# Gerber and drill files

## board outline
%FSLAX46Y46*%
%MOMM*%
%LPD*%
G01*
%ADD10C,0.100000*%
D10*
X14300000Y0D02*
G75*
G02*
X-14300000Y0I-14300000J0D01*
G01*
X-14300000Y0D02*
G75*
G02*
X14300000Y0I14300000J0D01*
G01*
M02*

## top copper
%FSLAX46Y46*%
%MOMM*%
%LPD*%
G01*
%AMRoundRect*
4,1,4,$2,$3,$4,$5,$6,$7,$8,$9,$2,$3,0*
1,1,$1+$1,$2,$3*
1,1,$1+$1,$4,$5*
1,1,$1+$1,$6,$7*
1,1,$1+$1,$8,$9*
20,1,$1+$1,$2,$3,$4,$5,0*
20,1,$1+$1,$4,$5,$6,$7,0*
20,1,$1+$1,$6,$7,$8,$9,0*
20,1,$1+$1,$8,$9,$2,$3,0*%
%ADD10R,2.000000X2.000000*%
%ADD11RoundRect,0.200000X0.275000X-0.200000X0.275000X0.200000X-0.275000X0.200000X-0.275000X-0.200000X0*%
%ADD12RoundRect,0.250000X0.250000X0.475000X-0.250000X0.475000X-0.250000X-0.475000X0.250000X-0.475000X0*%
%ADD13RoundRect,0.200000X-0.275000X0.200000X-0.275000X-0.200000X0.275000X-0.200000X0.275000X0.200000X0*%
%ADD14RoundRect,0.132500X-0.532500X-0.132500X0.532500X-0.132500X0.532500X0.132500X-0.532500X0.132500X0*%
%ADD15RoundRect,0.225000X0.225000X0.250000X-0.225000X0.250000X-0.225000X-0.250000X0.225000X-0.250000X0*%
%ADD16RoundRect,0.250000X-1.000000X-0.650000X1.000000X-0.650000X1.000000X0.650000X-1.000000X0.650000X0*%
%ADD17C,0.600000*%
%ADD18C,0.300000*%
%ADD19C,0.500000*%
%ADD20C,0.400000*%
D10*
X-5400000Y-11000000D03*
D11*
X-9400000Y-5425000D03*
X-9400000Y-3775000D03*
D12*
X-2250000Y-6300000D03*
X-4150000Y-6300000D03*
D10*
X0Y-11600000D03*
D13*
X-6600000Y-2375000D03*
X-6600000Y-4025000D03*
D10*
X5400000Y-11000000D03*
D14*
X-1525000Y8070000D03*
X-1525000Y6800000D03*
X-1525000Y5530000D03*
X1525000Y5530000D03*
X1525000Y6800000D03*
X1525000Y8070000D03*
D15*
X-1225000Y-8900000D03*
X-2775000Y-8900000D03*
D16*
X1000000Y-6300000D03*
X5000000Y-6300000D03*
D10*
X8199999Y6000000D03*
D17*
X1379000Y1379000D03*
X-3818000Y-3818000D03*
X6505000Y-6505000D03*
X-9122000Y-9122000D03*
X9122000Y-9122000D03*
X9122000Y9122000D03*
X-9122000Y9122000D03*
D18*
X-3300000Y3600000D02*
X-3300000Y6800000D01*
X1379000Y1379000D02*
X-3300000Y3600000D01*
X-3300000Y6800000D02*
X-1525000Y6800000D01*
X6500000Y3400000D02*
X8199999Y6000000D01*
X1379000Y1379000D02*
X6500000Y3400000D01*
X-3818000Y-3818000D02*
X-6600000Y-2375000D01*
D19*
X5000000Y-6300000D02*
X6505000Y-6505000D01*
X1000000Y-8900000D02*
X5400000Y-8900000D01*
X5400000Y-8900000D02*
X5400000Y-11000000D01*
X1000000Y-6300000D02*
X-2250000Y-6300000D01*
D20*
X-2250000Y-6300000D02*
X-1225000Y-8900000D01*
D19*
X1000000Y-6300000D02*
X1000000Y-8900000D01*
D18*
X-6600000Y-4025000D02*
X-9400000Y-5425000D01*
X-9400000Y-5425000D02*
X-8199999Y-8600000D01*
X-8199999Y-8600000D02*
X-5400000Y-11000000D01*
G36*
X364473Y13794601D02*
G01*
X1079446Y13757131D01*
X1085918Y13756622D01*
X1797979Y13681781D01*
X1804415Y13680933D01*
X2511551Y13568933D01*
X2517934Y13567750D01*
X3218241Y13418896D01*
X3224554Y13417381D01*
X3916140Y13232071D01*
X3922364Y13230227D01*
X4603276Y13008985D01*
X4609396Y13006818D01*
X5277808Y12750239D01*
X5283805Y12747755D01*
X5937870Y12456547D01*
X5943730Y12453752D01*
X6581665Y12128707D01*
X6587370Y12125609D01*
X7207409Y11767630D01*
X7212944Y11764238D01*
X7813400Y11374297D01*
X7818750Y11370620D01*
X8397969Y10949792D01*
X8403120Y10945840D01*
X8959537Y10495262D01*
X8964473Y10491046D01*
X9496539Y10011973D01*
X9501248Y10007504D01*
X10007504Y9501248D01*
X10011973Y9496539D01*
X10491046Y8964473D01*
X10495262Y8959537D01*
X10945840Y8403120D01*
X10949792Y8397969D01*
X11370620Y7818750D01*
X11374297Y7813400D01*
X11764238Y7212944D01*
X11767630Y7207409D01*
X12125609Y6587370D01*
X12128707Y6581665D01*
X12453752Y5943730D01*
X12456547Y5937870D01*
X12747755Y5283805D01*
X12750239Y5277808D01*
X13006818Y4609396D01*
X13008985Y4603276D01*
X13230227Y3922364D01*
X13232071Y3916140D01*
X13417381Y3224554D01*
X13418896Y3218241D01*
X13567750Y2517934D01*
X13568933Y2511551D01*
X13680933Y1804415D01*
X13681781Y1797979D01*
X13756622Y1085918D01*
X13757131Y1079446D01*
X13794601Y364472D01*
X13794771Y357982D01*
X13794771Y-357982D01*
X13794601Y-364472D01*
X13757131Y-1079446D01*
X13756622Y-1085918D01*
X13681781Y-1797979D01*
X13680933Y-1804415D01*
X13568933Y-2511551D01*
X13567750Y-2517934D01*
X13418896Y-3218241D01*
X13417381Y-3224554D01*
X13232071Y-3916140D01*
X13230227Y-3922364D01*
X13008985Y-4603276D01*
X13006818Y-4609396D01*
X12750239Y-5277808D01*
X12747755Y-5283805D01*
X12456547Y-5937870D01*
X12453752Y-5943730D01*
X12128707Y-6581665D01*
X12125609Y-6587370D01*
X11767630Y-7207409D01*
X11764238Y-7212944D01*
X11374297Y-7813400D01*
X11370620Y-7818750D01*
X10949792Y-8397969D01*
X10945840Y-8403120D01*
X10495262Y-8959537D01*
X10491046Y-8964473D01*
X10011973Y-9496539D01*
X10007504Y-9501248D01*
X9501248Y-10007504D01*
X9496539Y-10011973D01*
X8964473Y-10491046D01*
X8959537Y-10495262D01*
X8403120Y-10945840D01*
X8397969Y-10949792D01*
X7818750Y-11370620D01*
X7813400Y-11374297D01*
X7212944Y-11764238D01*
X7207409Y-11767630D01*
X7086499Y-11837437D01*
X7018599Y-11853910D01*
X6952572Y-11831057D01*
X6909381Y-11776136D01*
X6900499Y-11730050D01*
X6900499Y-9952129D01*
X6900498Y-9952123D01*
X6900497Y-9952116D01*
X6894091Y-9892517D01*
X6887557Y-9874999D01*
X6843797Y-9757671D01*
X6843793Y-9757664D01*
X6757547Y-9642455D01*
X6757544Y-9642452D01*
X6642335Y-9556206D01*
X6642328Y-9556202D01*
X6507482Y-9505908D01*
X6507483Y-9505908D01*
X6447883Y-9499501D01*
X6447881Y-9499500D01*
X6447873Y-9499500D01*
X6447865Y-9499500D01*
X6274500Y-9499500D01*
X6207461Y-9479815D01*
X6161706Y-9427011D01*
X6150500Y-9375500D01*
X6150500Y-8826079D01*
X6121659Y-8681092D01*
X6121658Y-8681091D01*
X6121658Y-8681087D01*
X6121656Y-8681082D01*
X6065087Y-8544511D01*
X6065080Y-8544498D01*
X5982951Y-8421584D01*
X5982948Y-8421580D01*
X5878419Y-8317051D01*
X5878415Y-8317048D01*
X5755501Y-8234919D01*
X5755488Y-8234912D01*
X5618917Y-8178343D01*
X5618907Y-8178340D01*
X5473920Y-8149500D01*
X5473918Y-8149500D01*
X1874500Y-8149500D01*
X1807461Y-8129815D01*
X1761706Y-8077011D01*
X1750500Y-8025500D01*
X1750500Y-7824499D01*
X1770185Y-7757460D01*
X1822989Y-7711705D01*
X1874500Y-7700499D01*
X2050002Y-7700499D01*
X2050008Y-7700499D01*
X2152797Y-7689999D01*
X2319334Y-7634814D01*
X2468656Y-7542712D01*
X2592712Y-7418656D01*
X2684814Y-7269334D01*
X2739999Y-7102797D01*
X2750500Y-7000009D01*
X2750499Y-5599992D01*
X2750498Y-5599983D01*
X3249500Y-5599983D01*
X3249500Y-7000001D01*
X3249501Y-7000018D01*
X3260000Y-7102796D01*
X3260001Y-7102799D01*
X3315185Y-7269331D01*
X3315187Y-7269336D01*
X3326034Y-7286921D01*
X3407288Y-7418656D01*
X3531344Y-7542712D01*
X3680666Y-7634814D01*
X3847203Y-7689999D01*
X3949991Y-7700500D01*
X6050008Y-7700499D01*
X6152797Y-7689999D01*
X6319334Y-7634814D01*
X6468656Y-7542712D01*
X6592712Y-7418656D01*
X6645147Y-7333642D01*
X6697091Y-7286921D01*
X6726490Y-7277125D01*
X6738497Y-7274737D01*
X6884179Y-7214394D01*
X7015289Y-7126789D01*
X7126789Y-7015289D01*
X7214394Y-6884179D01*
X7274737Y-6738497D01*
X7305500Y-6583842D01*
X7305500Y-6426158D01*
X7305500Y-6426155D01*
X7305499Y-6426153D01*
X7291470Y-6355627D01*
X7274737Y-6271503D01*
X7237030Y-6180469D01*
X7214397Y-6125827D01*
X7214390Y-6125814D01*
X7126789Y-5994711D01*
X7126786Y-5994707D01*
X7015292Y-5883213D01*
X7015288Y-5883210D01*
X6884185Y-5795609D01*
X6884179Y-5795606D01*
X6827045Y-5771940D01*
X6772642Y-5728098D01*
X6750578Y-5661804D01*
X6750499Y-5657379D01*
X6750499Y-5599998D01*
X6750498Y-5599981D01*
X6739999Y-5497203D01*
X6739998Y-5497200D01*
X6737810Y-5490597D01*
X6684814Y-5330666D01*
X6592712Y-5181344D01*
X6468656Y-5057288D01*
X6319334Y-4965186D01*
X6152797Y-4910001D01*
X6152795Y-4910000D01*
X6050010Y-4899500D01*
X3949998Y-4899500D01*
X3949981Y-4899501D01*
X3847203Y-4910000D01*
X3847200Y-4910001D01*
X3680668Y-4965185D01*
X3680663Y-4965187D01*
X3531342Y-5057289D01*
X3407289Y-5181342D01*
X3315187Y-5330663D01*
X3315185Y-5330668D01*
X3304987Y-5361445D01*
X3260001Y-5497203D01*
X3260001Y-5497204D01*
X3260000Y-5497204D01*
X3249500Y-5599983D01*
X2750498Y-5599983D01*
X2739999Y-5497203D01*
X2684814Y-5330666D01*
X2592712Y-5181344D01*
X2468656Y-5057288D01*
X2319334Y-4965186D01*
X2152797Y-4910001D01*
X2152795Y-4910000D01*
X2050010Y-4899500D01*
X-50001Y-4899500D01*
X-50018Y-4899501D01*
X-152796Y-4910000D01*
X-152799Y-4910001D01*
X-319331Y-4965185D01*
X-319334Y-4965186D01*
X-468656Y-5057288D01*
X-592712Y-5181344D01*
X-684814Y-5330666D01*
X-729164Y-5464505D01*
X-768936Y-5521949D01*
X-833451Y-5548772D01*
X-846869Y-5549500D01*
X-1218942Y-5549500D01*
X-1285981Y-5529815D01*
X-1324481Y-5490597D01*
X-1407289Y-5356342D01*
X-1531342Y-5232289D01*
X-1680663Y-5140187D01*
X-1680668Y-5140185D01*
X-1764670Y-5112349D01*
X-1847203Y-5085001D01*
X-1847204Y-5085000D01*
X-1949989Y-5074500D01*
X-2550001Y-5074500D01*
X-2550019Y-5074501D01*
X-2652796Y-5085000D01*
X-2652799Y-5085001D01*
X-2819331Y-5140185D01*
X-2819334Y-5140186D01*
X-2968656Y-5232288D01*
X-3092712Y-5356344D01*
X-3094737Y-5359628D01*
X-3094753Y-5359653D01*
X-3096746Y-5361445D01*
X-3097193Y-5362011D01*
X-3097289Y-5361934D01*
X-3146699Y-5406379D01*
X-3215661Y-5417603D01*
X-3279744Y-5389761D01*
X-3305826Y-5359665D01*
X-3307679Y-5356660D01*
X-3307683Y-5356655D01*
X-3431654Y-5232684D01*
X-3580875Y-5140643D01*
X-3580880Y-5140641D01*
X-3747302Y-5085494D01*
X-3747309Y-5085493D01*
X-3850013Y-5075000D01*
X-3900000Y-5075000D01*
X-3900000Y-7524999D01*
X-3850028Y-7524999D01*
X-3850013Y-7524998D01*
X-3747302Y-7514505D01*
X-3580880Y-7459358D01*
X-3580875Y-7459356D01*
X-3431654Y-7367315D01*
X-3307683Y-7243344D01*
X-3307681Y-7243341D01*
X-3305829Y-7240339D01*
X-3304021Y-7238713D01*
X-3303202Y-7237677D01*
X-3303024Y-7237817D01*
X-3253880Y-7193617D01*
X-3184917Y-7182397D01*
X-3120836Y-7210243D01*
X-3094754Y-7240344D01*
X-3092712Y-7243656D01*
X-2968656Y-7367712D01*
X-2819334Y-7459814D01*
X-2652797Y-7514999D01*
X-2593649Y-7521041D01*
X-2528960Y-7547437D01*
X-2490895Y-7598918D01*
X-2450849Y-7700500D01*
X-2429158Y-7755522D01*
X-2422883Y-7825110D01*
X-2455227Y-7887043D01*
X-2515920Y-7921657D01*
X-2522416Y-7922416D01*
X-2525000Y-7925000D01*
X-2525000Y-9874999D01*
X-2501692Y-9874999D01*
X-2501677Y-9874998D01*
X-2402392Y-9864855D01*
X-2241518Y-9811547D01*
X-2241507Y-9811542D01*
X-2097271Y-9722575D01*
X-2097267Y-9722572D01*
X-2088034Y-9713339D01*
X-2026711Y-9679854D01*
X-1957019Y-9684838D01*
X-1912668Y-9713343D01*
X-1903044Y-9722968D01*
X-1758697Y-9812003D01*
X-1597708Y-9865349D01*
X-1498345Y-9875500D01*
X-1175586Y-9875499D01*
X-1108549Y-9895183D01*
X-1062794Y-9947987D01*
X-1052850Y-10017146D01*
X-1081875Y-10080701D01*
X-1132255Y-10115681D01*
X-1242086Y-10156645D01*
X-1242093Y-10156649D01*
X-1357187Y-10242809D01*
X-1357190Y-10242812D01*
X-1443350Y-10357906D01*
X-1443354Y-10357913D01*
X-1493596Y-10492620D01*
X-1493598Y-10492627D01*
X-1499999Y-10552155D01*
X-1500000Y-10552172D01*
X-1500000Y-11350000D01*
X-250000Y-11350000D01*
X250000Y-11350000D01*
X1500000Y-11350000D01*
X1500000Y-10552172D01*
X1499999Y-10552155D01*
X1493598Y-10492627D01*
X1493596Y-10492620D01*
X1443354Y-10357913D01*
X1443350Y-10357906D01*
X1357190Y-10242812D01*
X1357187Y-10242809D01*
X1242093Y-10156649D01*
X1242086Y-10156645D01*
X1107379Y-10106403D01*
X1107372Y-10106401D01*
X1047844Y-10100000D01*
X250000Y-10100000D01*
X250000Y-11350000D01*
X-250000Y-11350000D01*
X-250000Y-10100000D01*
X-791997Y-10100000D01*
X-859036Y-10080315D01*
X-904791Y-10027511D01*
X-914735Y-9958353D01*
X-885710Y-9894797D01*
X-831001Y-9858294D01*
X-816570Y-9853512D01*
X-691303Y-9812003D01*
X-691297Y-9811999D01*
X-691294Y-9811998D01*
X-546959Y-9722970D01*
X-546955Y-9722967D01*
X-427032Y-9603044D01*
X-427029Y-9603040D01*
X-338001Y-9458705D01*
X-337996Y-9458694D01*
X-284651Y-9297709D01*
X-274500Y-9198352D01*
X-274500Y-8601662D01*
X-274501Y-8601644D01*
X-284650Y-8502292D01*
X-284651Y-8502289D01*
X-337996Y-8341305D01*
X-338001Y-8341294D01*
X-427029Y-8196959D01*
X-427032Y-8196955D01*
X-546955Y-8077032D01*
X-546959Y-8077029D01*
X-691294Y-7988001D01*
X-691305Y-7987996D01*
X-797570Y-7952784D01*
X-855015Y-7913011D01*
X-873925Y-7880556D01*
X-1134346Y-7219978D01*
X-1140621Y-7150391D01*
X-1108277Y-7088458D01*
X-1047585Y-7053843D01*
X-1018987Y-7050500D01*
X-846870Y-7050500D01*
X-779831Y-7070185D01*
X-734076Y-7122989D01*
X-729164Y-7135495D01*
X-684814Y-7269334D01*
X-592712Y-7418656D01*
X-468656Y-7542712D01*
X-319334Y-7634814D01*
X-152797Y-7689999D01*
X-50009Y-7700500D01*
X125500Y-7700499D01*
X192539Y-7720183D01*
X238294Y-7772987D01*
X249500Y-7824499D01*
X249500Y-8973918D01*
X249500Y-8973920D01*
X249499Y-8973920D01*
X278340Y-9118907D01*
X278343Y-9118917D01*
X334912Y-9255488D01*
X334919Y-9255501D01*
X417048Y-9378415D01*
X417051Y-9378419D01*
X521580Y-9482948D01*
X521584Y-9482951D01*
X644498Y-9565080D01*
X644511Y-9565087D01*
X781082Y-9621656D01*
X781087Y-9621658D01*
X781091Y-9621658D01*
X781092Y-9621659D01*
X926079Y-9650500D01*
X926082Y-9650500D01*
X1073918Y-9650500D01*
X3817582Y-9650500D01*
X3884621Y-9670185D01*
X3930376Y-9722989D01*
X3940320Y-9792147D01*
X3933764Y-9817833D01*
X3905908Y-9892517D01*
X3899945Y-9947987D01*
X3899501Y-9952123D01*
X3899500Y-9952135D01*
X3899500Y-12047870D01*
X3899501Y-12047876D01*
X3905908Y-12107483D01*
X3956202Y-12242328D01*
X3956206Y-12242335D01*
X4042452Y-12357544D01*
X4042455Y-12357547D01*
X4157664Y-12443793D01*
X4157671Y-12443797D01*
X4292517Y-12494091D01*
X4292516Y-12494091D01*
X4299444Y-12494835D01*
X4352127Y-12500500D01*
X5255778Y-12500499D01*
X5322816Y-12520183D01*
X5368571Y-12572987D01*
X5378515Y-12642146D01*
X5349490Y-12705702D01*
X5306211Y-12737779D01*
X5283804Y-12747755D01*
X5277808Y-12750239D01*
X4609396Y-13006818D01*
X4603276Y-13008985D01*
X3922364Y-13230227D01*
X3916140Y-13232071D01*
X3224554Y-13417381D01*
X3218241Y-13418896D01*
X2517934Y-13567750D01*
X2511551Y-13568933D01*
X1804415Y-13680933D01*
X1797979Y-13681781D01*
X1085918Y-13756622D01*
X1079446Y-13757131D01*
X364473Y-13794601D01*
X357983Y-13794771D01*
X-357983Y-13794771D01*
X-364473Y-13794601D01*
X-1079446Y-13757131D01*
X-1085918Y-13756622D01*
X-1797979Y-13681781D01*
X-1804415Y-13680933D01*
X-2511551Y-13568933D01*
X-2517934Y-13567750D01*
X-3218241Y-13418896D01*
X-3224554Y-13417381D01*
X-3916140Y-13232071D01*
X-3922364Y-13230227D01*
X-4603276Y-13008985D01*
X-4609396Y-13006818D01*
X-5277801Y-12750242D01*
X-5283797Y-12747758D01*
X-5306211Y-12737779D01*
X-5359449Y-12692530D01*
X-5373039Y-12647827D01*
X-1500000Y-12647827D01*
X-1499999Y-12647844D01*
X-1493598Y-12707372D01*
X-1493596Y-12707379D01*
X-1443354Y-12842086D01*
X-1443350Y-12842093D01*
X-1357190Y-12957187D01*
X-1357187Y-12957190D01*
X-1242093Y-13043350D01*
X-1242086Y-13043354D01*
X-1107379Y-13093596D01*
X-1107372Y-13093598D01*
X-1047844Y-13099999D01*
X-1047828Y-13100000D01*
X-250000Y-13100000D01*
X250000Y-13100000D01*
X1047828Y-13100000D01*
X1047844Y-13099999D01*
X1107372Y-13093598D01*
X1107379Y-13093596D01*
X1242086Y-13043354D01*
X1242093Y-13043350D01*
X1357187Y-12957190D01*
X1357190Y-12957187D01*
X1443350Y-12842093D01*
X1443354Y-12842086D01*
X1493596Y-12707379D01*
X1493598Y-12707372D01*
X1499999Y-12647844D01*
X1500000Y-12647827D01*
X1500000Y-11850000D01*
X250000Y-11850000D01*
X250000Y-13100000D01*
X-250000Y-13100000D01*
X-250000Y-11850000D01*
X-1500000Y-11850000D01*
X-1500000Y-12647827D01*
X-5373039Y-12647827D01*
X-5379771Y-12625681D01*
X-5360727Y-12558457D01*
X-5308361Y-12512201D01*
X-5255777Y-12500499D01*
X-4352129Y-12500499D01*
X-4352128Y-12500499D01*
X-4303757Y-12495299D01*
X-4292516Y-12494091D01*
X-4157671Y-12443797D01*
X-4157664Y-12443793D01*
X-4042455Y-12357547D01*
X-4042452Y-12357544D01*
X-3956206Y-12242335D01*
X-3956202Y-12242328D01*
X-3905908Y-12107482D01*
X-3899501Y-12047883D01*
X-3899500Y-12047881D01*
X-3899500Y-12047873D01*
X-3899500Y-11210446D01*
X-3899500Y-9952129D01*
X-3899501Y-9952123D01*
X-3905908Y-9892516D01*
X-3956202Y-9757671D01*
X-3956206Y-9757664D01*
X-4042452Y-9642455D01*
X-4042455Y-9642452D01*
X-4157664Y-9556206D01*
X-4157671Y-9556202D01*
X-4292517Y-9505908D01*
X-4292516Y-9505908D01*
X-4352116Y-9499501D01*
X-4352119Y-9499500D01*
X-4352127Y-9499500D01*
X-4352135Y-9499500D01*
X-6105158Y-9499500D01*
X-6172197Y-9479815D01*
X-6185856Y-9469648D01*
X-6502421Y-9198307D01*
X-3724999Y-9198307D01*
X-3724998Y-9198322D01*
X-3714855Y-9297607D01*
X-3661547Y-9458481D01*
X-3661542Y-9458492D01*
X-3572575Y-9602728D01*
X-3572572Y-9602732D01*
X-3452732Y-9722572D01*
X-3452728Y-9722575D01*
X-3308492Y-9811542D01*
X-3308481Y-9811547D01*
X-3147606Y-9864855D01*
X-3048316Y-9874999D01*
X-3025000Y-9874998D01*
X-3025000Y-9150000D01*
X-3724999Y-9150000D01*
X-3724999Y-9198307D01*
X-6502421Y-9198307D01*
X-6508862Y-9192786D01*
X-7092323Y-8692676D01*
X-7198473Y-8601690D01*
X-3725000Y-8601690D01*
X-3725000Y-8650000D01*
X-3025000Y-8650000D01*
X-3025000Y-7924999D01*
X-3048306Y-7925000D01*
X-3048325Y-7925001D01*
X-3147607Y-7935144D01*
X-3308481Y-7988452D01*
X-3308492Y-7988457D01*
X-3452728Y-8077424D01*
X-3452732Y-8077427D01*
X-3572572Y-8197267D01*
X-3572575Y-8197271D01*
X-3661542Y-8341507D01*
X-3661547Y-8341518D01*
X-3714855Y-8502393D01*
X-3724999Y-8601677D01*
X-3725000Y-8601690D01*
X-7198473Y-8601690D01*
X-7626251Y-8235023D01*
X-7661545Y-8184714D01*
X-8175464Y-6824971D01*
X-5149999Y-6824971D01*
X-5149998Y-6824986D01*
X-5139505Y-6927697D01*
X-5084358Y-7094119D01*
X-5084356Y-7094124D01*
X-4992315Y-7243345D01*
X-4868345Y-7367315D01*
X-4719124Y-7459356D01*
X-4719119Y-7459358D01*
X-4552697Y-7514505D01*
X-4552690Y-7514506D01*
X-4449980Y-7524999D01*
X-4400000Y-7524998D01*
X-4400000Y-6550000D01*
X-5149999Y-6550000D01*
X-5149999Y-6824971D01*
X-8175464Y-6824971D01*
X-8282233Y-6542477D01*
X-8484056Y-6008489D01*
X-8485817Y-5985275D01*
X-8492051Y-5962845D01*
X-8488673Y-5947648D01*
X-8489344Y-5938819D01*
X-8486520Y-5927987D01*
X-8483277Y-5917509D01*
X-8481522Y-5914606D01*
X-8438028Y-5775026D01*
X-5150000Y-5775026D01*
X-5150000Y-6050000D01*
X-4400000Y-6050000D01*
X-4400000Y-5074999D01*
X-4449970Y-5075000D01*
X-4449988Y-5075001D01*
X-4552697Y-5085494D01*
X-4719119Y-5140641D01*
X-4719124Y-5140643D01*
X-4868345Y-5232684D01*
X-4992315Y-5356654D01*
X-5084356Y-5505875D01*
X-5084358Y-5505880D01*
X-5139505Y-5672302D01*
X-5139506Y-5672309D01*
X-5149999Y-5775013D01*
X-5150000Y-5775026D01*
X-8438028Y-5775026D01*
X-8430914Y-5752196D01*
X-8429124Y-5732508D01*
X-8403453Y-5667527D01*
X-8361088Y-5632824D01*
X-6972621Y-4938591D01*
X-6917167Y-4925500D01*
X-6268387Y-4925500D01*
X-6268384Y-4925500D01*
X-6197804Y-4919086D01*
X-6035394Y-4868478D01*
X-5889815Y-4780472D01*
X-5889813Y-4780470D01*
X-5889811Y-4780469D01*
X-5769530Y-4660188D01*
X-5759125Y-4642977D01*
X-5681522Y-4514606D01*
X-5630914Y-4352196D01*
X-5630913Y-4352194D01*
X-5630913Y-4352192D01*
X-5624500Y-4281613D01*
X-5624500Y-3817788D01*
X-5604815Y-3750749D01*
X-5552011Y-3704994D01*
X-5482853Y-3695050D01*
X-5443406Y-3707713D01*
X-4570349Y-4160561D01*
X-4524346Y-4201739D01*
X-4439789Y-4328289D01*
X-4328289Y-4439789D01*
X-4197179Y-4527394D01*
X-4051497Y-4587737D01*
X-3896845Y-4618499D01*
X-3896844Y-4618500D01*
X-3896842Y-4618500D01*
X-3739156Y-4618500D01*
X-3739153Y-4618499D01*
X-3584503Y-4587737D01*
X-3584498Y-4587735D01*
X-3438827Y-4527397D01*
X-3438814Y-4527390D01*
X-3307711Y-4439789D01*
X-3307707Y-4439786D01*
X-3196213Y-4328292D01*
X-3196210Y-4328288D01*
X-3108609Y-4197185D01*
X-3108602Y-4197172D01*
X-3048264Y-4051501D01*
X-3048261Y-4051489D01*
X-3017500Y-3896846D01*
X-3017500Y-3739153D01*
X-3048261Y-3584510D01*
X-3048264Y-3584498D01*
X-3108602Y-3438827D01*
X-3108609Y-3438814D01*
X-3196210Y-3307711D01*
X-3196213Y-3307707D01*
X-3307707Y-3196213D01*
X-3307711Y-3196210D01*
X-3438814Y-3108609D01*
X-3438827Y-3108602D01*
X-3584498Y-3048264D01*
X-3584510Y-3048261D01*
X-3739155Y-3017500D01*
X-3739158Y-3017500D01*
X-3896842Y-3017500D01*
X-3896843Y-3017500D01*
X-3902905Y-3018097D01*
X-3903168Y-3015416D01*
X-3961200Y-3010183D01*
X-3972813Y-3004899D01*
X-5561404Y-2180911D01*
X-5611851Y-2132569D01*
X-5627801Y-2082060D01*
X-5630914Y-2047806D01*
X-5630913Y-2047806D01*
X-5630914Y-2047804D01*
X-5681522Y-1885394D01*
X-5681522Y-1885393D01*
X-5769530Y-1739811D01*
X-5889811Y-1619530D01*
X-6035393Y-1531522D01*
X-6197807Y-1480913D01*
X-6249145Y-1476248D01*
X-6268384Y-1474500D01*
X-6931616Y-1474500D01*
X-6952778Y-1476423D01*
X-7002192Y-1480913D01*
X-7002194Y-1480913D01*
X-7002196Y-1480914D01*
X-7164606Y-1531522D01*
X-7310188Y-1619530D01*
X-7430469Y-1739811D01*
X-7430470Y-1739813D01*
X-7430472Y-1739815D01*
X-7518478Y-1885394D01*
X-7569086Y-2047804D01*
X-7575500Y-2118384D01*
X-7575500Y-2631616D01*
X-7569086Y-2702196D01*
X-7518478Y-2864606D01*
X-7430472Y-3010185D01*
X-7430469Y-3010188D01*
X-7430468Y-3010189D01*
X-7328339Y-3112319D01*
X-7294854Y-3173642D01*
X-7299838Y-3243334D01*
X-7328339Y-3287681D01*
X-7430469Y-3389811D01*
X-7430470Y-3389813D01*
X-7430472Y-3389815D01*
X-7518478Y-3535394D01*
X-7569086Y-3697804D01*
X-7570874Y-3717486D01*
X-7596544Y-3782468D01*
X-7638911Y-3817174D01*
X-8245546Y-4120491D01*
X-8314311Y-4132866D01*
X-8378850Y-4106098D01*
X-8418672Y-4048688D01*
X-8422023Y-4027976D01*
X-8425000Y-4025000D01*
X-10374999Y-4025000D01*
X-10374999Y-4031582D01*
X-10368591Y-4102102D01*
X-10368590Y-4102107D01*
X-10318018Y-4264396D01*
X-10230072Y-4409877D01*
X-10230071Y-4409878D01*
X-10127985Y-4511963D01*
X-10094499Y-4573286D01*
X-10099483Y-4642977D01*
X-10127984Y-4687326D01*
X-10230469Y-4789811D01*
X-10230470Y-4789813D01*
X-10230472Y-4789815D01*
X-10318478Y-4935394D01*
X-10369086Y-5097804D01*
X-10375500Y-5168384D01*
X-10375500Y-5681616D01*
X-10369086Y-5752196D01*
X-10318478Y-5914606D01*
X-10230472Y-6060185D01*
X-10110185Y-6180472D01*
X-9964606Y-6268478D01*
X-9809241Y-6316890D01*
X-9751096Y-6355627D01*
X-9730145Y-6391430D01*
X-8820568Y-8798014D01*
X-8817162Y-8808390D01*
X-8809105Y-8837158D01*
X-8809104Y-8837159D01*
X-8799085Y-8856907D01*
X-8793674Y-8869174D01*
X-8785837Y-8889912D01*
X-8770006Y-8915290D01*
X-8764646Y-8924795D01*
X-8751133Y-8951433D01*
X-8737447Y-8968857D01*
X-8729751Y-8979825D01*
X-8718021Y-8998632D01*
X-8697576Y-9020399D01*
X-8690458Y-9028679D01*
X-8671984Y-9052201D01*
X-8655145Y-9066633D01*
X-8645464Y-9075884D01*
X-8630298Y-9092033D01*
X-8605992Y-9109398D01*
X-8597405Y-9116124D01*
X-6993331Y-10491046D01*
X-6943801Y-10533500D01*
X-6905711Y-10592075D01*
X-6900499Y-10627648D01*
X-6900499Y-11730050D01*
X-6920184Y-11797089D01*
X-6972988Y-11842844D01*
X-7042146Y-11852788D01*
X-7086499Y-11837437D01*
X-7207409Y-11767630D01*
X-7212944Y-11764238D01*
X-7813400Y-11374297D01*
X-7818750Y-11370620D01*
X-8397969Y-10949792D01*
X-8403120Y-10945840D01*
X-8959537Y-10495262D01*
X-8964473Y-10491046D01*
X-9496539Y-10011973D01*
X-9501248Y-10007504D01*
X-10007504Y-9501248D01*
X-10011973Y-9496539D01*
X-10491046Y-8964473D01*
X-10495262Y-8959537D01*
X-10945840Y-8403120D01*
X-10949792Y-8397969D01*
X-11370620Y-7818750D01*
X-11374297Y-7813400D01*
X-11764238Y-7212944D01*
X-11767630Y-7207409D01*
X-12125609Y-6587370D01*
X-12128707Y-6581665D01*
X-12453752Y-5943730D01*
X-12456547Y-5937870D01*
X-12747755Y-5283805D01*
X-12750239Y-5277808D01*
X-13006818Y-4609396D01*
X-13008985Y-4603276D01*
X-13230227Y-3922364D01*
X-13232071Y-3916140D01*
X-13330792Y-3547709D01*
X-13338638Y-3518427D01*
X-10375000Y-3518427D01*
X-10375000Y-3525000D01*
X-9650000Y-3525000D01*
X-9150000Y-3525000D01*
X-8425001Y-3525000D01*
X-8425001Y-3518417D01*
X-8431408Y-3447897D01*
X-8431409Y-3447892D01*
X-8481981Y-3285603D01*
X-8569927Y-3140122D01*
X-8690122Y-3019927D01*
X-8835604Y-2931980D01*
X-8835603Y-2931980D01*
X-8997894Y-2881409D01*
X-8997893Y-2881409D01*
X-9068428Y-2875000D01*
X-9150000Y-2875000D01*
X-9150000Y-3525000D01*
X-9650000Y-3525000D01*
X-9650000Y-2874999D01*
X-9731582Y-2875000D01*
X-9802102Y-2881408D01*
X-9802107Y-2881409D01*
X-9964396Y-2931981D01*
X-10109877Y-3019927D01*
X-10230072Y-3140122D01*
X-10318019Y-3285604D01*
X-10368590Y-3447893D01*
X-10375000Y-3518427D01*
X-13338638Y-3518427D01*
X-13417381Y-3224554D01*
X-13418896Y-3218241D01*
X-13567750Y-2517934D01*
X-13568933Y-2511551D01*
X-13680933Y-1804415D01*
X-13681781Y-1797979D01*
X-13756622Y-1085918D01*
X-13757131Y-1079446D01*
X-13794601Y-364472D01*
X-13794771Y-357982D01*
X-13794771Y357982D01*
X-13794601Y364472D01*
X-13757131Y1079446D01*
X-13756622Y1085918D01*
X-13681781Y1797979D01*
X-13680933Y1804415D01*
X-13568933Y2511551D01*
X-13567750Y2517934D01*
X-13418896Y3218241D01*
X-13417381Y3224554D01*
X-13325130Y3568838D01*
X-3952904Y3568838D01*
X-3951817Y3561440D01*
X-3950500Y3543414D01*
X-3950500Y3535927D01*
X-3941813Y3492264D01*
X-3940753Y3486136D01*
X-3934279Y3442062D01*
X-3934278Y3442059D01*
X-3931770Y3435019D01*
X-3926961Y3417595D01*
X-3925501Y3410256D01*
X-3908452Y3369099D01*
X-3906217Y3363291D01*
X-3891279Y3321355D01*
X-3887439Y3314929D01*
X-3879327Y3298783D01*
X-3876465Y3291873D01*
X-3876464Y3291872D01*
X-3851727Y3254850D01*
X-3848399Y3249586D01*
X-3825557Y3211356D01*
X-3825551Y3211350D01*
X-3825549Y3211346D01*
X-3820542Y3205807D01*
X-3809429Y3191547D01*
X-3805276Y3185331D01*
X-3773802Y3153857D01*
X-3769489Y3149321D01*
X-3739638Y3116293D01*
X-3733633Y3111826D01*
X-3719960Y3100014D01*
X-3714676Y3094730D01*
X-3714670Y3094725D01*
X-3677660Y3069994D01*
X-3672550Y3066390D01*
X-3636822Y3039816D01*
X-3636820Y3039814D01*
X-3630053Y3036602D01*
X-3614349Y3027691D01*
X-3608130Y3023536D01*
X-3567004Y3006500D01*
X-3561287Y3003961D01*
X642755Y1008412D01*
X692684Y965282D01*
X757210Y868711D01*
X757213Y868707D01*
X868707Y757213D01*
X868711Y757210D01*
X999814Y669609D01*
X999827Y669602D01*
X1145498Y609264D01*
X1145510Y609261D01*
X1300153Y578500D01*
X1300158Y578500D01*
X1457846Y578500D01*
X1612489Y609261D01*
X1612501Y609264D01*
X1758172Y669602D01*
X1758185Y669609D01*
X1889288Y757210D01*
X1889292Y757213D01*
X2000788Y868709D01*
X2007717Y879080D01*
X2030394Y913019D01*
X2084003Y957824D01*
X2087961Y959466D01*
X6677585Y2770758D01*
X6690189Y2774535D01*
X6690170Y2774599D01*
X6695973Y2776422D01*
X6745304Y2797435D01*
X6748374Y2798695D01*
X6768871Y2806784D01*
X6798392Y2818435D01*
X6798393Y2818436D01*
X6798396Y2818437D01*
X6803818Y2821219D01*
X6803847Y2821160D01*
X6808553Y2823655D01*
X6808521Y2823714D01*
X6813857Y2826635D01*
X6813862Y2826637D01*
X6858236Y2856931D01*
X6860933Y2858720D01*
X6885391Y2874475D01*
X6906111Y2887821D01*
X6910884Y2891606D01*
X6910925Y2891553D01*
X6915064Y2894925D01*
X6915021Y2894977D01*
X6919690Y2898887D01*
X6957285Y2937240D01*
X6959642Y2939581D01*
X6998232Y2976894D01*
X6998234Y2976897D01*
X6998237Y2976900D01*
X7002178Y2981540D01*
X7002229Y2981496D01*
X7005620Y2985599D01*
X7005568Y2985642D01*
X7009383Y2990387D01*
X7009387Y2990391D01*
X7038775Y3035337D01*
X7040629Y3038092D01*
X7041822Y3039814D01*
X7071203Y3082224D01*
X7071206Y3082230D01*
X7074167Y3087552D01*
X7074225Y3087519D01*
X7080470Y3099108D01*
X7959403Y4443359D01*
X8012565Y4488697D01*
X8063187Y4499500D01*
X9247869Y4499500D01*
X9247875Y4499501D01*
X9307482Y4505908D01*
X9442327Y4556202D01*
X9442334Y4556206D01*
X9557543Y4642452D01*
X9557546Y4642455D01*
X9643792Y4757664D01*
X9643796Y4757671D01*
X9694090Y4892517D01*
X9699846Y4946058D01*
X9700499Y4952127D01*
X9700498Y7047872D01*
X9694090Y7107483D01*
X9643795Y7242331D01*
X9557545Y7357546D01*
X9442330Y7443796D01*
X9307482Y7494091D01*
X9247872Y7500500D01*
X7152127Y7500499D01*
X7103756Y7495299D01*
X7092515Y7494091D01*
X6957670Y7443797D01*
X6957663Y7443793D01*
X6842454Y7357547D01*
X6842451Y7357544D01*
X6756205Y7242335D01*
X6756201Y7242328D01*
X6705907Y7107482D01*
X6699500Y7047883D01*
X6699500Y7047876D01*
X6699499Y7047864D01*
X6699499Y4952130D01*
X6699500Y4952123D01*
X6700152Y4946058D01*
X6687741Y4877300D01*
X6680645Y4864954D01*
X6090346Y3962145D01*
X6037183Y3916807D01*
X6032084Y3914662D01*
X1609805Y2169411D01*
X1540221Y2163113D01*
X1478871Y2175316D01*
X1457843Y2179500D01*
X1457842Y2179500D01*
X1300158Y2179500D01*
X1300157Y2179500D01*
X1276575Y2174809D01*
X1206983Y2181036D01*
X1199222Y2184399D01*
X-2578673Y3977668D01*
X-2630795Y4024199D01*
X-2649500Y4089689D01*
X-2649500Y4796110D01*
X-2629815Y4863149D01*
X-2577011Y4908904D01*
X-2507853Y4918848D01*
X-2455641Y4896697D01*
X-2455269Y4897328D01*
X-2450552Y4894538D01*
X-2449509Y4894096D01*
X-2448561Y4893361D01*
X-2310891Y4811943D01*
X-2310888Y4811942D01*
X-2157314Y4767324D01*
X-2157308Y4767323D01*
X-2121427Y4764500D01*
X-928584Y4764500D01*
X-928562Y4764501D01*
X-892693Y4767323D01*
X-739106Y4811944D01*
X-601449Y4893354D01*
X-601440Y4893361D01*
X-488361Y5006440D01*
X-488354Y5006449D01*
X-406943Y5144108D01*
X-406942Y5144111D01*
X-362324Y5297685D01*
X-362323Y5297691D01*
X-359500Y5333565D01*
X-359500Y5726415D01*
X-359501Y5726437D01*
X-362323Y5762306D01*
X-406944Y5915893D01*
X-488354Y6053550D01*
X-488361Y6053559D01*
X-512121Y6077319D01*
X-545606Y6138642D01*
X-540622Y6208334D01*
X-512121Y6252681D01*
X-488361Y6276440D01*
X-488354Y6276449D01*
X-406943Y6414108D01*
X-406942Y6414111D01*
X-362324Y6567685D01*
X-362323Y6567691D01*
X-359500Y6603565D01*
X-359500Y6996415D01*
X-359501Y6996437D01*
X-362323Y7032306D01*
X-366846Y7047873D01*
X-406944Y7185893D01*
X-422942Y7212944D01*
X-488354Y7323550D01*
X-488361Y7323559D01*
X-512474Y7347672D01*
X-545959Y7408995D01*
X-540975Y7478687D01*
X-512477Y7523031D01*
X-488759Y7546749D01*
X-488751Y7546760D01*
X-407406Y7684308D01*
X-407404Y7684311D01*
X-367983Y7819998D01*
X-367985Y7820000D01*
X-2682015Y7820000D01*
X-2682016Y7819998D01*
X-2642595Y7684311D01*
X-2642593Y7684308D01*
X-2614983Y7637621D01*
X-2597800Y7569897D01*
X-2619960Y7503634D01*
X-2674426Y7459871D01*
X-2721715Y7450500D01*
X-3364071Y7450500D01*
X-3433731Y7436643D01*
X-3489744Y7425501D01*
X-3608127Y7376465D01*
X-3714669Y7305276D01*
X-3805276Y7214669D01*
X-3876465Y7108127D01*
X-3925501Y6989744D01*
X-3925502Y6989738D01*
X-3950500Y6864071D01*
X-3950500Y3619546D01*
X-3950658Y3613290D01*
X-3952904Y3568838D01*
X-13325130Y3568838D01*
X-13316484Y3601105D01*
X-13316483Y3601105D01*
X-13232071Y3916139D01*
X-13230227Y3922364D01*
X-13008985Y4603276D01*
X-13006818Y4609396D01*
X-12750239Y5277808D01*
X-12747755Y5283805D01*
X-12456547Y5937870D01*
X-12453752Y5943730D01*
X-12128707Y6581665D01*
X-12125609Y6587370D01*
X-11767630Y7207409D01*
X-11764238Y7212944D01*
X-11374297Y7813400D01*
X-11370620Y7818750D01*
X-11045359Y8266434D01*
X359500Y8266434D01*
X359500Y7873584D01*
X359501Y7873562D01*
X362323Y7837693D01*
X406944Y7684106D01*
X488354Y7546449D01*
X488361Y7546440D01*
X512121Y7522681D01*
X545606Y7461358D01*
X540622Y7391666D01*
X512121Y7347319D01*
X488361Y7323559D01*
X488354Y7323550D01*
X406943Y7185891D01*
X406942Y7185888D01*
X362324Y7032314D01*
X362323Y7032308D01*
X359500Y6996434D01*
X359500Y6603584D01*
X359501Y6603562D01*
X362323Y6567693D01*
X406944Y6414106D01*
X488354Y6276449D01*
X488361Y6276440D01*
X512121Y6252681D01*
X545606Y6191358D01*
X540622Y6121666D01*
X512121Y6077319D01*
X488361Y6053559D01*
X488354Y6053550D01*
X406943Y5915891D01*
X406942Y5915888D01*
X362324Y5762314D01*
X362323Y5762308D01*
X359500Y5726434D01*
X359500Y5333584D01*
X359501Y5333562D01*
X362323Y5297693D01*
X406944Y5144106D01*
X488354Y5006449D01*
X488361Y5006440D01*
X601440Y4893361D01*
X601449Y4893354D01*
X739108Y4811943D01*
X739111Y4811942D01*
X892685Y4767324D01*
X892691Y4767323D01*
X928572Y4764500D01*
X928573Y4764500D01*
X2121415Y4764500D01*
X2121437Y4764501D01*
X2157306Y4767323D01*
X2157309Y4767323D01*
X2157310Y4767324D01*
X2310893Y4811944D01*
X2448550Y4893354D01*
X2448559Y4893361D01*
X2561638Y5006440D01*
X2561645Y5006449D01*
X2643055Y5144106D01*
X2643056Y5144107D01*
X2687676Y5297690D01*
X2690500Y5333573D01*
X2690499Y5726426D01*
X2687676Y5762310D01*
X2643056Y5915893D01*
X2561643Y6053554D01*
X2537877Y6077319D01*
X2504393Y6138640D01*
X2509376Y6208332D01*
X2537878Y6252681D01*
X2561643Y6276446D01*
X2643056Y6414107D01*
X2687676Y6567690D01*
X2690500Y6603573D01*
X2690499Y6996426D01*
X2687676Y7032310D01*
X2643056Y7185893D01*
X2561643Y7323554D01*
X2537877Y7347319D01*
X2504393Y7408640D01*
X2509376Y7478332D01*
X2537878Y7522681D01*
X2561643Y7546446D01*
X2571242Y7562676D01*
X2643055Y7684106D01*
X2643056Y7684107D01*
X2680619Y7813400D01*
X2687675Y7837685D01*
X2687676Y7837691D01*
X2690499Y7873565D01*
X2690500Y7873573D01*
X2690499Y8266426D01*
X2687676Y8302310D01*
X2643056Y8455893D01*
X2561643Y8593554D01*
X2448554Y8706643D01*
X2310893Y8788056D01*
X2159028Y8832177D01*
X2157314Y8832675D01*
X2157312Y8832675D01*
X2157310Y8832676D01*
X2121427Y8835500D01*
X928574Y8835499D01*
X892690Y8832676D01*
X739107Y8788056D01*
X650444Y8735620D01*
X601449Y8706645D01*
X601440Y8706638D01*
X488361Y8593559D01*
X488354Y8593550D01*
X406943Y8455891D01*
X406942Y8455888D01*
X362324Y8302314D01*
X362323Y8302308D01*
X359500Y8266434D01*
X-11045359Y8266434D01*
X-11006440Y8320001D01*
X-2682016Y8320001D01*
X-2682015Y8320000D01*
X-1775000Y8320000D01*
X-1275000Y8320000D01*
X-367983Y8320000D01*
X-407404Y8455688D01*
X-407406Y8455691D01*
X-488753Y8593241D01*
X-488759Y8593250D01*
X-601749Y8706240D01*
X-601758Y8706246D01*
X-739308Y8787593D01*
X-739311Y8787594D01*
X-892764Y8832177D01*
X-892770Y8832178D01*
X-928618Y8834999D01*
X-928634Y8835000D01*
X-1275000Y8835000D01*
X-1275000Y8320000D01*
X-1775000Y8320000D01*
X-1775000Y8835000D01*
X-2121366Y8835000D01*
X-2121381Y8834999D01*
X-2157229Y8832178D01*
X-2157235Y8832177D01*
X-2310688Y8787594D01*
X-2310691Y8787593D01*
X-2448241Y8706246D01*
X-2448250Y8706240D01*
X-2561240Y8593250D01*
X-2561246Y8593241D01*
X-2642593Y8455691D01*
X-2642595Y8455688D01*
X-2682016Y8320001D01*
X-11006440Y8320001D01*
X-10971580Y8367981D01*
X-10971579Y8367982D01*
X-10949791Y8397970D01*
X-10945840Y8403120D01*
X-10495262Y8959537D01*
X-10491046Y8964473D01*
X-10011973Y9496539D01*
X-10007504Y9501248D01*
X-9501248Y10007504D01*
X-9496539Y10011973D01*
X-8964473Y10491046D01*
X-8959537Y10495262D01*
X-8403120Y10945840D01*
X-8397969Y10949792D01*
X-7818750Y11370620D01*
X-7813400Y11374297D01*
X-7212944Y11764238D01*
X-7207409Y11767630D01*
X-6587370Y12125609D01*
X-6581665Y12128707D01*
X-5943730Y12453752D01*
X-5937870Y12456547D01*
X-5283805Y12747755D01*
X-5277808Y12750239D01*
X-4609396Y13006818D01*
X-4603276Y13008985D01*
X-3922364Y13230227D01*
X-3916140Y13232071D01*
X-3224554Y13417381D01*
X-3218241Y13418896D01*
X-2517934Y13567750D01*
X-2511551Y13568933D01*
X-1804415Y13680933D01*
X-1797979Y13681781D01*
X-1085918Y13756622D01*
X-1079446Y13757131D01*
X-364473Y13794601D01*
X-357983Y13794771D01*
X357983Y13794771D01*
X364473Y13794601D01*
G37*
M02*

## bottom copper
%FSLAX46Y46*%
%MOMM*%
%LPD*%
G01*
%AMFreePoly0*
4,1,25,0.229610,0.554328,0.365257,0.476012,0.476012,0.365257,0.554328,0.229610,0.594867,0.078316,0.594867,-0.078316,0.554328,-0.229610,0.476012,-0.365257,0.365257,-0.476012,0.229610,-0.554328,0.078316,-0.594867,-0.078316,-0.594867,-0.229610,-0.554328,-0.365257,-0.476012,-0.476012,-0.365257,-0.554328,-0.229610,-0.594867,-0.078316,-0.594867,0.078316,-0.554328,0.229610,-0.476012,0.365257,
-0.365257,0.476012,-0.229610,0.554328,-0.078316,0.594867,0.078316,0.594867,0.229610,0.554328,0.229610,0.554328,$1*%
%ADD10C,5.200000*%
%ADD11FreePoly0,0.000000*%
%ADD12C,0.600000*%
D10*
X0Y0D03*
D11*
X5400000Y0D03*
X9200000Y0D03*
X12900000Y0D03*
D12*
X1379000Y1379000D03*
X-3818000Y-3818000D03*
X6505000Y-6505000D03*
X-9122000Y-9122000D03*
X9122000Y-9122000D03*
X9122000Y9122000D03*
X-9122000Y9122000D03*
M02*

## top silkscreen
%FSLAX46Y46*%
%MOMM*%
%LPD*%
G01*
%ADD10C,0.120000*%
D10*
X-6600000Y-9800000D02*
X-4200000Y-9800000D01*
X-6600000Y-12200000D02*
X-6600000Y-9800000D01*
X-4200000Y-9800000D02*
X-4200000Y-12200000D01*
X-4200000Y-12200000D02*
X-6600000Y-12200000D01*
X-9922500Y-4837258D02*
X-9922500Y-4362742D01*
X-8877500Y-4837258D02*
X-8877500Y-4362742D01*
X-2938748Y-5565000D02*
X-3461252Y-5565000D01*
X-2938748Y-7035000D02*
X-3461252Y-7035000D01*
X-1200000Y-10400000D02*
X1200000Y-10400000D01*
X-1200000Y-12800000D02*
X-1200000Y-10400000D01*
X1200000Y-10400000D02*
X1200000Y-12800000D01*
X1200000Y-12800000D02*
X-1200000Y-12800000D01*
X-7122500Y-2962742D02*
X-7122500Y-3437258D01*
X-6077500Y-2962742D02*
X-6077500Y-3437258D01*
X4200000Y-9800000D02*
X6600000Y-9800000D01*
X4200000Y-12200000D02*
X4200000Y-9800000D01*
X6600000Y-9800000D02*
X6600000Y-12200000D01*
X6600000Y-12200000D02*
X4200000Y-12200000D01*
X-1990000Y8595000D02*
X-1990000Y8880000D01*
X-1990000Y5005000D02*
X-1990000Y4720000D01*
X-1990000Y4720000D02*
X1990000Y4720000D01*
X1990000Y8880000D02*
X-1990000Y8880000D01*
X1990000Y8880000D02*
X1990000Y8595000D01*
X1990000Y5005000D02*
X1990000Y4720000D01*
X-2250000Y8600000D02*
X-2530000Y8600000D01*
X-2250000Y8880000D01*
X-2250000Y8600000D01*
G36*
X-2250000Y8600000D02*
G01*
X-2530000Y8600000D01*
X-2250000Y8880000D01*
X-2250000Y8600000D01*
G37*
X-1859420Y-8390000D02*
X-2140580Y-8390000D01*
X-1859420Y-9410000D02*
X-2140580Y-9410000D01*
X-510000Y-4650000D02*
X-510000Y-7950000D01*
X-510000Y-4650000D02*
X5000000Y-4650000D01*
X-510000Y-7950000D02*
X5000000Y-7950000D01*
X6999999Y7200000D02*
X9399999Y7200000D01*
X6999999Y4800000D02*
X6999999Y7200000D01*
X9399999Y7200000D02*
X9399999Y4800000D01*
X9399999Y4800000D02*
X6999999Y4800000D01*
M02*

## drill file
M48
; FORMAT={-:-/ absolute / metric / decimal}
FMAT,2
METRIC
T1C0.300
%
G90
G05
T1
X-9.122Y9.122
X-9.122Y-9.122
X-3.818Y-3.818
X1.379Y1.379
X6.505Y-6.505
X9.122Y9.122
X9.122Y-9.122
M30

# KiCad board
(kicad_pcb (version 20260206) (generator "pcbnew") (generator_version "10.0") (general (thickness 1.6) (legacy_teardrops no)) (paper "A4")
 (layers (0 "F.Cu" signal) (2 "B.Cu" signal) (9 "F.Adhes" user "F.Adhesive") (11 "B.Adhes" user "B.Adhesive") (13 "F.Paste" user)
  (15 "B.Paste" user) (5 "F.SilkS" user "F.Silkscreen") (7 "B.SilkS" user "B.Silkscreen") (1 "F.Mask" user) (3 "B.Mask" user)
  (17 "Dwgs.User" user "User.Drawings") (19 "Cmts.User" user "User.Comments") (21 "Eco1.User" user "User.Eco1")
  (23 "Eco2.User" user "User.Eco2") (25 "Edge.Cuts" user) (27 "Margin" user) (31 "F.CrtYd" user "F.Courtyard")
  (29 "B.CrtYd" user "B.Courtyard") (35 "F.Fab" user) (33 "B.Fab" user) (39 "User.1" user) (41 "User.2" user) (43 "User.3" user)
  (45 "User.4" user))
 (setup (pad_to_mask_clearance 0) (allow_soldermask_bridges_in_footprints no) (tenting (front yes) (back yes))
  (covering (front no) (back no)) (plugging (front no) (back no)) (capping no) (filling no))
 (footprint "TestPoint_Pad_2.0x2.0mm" (layer "F.Cu") (at -5.4 11)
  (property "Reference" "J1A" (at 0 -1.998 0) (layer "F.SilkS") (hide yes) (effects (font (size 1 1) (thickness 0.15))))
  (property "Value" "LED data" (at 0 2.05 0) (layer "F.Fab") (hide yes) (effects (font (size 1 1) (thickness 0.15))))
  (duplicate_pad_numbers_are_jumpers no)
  (fp_line (start -1.2 -1.2) (end 1.2 -1.2) (stroke (width 0.12) (type solid)) (layer "F.SilkS"))
  (fp_line (start -1.2 1.2) (end -1.2 -1.2) (stroke (width 0.12) (type solid)) (layer "F.SilkS"))
  (fp_line (start 1.2 -1.2) (end 1.2 1.2) (stroke (width 0.12) (type solid)) (layer "F.SilkS"))
  (fp_line (start 1.2 1.2) (end -1.2 1.2) (stroke (width 0.12) (type solid)) (layer "F.SilkS"))
  (pad "1" smd rect (at 0 0) (size 2 2) (layers "F.Cu" "F.Mask") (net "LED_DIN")))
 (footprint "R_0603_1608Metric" (layer "F.Cu") (at -9.4 4.6 90)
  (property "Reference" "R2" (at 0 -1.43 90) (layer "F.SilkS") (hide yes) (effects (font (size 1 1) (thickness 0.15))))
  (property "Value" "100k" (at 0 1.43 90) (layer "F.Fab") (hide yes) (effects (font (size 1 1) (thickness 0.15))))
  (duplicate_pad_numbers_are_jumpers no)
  (fp_line (start -0.237258 -0.5225) (end 0.237258 -0.5225) (stroke (width 0.12) (type solid)) (layer "F.SilkS"))
  (fp_line (start -0.237258 0.5225) (end 0.237258 0.5225) (stroke (width 0.12) (type solid)) (layer "F.SilkS"))
  (pad "1" smd roundrect (at -0.825 0 90) (size 0.8 0.95) (layers "F.Cu" "F.Mask" "F.Paste") (roundrect_rratio 0.25) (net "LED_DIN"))
  (pad "2" smd roundrect (at 0.825 0 90) (size 0.8 0.95) (layers "F.Cu" "F.Mask" "F.Paste") (roundrect_rratio 0.25) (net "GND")))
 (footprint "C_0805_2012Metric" (layer "F.Cu") (at -3.2 6.3 180)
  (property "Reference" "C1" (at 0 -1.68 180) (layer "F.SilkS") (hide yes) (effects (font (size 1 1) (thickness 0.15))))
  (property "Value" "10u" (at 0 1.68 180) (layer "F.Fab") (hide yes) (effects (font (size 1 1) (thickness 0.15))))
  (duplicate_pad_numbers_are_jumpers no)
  (fp_line (start -0.261252 0.735) (end 0.261252 0.735) (stroke (width 0.12) (type solid)) (layer "F.SilkS"))
  (fp_line (start -0.261252 -0.735) (end 0.261252 -0.735) (stroke (width 0.12) (type solid)) (layer "F.SilkS"))
  (pad "1" smd roundrect (at -0.95 0 180) (size 1 1.45) (layers "F.Cu" "F.Mask" "F.Paste") (roundrect_rratio 0.25) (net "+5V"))
  (pad "2" smd roundrect (at 0.95 0 180) (size 1 1.45) (layers "F.Cu" "F.Mask" "F.Paste") (roundrect_rratio 0.25) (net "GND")))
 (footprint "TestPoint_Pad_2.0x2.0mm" (layer "F.Cu") (at 0 11.6)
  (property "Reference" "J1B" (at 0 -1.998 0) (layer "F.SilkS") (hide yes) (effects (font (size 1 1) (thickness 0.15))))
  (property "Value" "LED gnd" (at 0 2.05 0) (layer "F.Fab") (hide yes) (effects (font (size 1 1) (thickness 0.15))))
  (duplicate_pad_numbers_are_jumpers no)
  (fp_line (start -1.2 -1.2) (end 1.2 -1.2) (stroke (width 0.12) (type solid)) (layer "F.SilkS"))
  (fp_line (start -1.2 1.2) (end -1.2 -1.2) (stroke (width 0.12) (type solid)) (layer "F.SilkS"))
  (fp_line (start 1.2 -1.2) (end 1.2 1.2) (stroke (width 0.12) (type solid)) (layer "F.SilkS"))
  (fp_line (start 1.2 1.2) (end -1.2 1.2) (stroke (width 0.12) (type solid)) (layer "F.SilkS"))
  (pad "1" smd rect (at 0 0) (size 2 2) (layers "F.Cu" "F.Mask") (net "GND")))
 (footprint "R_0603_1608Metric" (layer "F.Cu") (at -6.6 3.2 -90)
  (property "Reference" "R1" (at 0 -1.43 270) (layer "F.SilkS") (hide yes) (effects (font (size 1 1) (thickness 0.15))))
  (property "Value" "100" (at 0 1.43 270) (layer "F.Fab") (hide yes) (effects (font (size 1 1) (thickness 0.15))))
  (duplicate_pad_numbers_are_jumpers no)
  (fp_line (start -0.237258 0.5225) (end 0.237258 0.5225) (stroke (width 0.12) (type solid)) (layer "F.SilkS"))
  (fp_line (start -0.237258 -0.5225) (end 0.237258 -0.5225) (stroke (width 0.12) (type solid)) (layer "F.SilkS"))
  (pad "1" smd roundrect (at -0.825 0 270) (size 0.8 0.95) (layers "F.Cu" "F.Mask" "F.Paste") (roundrect_rratio 0.25) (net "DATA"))
  (pad "2" smd roundrect (at 0.825 0 270) (size 0.8 0.95) (layers "F.Cu" "F.Mask" "F.Paste") (roundrect_rratio 0.25) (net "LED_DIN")))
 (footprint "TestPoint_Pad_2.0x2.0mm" (layer "F.Cu") (at 5.4 11)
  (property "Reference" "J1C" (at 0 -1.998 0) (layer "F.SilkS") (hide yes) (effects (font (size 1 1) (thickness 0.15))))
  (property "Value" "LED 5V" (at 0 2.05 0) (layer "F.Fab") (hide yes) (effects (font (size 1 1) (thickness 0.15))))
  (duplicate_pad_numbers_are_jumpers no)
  (fp_line (start -1.2 -1.2) (end 1.2 -1.2) (stroke (width 0.12) (type solid)) (layer "F.SilkS"))
  (fp_line (start -1.2 1.2) (end -1.2 -1.2) (stroke (width 0.12) (type solid)) (layer "F.SilkS"))
  (fp_line (start 1.2 -1.2) (end 1.2 1.2) (stroke (width 0.12) (type solid)) (layer "F.SilkS"))
  (fp_line (start 1.2 1.2) (end -1.2 1.2) (stroke (width 0.12) (type solid)) (layer "F.SilkS"))
  (pad "1" smd rect (at 0 0) (size 2 2) (layers "F.Cu" "F.Mask") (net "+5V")))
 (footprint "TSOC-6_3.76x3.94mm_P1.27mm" (layer "F.Cu") (at 0 -6.8)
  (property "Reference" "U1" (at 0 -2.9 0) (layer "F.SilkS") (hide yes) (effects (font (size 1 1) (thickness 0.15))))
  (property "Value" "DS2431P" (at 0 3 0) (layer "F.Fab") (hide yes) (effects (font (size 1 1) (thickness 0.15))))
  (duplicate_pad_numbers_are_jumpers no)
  (fp_line (start -1.99 -1.795) (end -1.99 -2.08) (stroke (width 0.12) (type solid)) (layer "F.SilkS"))
  (fp_line (start -1.99 1.795) (end -1.99 2.08) (stroke (width 0.12) (type solid)) (layer "F.SilkS"))
  (fp_line (start -1.99 2.08) (end 1.99 2.08) (stroke (width 0.12) (type solid)) (layer "F.SilkS"))
  (fp_line (start 1.99 -2.08) (end -1.99 -2.08) (stroke (width 0.12) (type solid)) (layer "F.SilkS"))
  (fp_line (start 1.99 -2.08) (end 1.99 -1.795) (stroke (width 0.12) (type solid)) (layer "F.SilkS"))
  (fp_line (start 1.99 1.795) (end 1.99 2.08) (stroke (width 0.12) (type solid)) (layer "F.SilkS"))
  (fp_poly
   (pts (xy -2.25 -1.8) (xy -2.53 -1.8) (xy -2.25 -2.08) (xy -2.25 -1.8)) (stroke (width 0.12) (type solid)) (fill yes) (layer "F.SilkS"))
  (pad "1" smd roundrect (at -1.525 -1.27) (size 1.33 0.53) (layers "F.Cu" "F.Mask" "F.Paste") (roundrect_rratio 0.25) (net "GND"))
  (pad "2" smd roundrect (at -1.525 0) (size 1.33 0.53) (layers "F.Cu" "F.Mask" "F.Paste") (roundrect_rratio 0.25) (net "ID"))
  (pad "3" smd roundrect (at -1.525 1.27) (size 1.33 0.53) (layers "F.Cu" "F.Mask" "F.Paste") (roundrect_rratio 0.25))
  (pad "4" smd roundrect (at 1.525 1.27) (size 1.33 0.53) (layers "F.Cu" "F.Mask" "F.Paste") (roundrect_rratio 0.25))
  (pad "5" smd roundrect (at 1.525 0) (size 1.33 0.53) (layers "F.Cu" "F.Mask" "F.Paste") (roundrect_rratio 0.25))
  (pad "6" smd roundrect (at 1.525 -1.27) (size 1.33 0.53) (layers "F.Cu" "F.Mask" "F.Paste") (roundrect_rratio 0.25)))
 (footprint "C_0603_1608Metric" (layer "F.Cu") (at -2 8.9 180)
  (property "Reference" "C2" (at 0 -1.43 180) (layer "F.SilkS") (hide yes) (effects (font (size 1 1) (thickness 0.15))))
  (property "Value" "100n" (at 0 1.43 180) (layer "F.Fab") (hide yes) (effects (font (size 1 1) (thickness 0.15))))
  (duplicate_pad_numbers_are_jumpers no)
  (fp_line (start -0.14058 0.51) (end 0.14058 0.51) (stroke (width 0.12) (type solid)) (layer "F.SilkS"))
  (fp_line (start -0.14058 -0.51) (end 0.14058 -0.51) (stroke (width 0.12) (type solid)) (layer "F.SilkS"))
  (pad "1" smd roundrect (at -0.775 0 180) (size 0.9 0.95) (layers "F.Cu" "F.Mask" "F.Paste") (roundrect_rratio 0.25) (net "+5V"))
  (pad "2" smd roundrect (at 0.775 0 180) (size 0.9 0.95) (layers "F.Cu" "F.Mask" "F.Paste") (roundrect_rratio 0.25) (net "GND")))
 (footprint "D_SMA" (layer "F.Cu") (at 3 6.3)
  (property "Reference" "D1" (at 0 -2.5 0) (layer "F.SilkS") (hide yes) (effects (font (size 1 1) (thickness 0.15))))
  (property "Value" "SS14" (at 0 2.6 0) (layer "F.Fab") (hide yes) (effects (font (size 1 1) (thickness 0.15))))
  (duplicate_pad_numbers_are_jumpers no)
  (fp_line (start -3.51 -1.65) (end -3.51 1.65) (stroke (width 0.12) (type solid)) (layer "F.SilkS"))
  (fp_line (start -3.51 -1.65) (end 2 -1.65) (stroke (width 0.12) (type solid)) (layer "F.SilkS"))
  (fp_line (start -3.51 1.65) (end 2 1.65) (stroke (width 0.12) (type solid)) (layer "F.SilkS"))
  (pad "1" smd roundrect (at -2 0) (size 2.5 1.8) (layers "F.Cu" "F.Mask" "F.Paste") (roundrect_rratio 0.1388888889) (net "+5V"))
  (pad "2" smd roundrect (at 2 0) (size 2.5 1.8) (layers "F.Cu" "F.Mask" "F.Paste") (roundrect_rratio 0.1388888889) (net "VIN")))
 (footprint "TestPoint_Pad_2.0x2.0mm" (layer "F.Cu") (at 8.199999 -6)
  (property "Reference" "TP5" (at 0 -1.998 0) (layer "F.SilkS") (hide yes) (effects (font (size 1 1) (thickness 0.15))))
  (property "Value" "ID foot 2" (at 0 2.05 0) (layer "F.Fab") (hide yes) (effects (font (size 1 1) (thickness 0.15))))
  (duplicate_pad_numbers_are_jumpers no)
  (fp_line (start -1.2 -1.2) (end 1.2 -1.2) (stroke (width 0.12) (type solid)) (layer "F.SilkS"))
  (fp_line (start -1.2 1.2) (end -1.2 -1.2) (stroke (width 0.12) (type solid)) (layer "F.SilkS"))
  (fp_line (start 1.2 -1.2) (end 1.2 1.2) (stroke (width 0.12) (type solid)) (layer "F.SilkS"))
  (fp_line (start 1.2 1.2) (end -1.2 1.2) (stroke (width 0.12) (type solid)) (layer "F.SilkS"))
  (pad "1" smd rect (at 0 0) (size 2 2) (layers "F.Cu" "F.Mask") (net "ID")))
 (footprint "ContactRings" (layer "B.Cu") (at 0 0)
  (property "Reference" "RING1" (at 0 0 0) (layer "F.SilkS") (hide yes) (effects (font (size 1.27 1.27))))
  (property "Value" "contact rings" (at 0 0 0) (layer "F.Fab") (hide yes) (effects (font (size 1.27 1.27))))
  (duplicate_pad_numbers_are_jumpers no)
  (pad "1" smd circle (at 0 0) (size 5.2 5.2) (layers "B.Cu" "B.Mask") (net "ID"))
  (pad "2" smd custom (at 5.4 0) (size 1.2 1.2) (layers "B.Cu" "B.Mask") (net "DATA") (options (clearance outline) (anchor circle))
   (primitives))
  (pad "3" smd custom (at 9.2 0) (size 1.2 1.2) (layers "B.Cu" "B.Mask") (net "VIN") (options (clearance outline) (anchor circle))
   (primitives))
  (pad "4" smd custom (at 12.9 0) (size 1.2 1.2) (layers "B.Cu" "B.Mask") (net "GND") (options (clearance outline) (anchor circle))
   (primitives)))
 (gr_circle (center 0 0) (end 14.3 0) (stroke (width 0.1) (type default)) (fill no) (layer "Edge.Cuts"))
 (segment (start -3.3 -3.6) (end -3.3 -6.8) (width 0.3) (layer "F.Cu") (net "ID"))
 (segment (start 1.379 -1.379) (end -3.3 -3.6) (width 0.3) (layer "F.Cu") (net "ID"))
 (segment (start -3.3 -6.8) (end -1.525 -6.8) (width 0.3) (layer "F.Cu") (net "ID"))
 (segment (start 6.5 -3.4) (end 8.199999 -6) (width 0.3) (layer "F.Cu") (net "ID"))
 (segment (start 1.379 -1.379) (end 6.5 -3.4) (width 0.3) (layer "F.Cu") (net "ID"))
 (via (at 1.379 -1.379) (size 0.6) (drill 0.3) (layers "F.Cu" "B.Cu") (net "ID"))
 (segment (start -3.818 3.818) (end -6.6 2.375) (width 0.3) (layer "F.Cu") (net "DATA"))
 (via (at -3.818 3.818) (size 0.6) (drill 0.3) (layers "F.Cu" "B.Cu") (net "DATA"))
 (segment (start 5 6.3) (end 6.505 6.505) (width 0.5) (layer "F.Cu") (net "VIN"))
 (via (at 6.505 6.505) (size 0.6) (drill 0.3) (layers "F.Cu" "B.Cu") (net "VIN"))
 (via (at -9.122 9.122) (size 0.6) (drill 0.3) (layers "F.Cu" "B.Cu") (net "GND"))
 (via (at 9.122 9.122) (size 0.6) (drill 0.3) (layers "F.Cu" "B.Cu") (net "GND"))
 (via (at 9.122 -9.122) (size 0.6) (drill 0.3) (layers "F.Cu" "B.Cu") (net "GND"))
 (via (at -9.122 -9.122) (size 0.6) (drill 0.3) (layers "F.Cu" "B.Cu") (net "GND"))
 (segment (start 1 8.9) (end 5.4 8.9) (width 0.5) (layer "F.Cu") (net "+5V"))
 (segment (start 5.4 8.9) (end 5.4 11) (width 0.5) (layer "F.Cu") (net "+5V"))
 (segment (start 1 6.3) (end -2.25 6.3) (width 0.5) (layer "F.Cu") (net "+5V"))
 (segment (start -2.25 6.3) (end -1.225 8.9) (width 0.4) (layer "F.Cu") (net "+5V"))
 (segment (start 1 6.3) (end 1 8.9) (width 0.5) (layer "F.Cu") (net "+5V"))
 (segment (start -6.6 4.025) (end -9.4 5.425) (width 0.3) (layer "F.Cu") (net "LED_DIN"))
 (segment (start -9.4 5.425) (end -8.199999 8.6) (width 0.3) (layer "F.Cu") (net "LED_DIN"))
 (segment (start -8.199999 8.6) (end -5.4 11) (width 0.3) (layer "F.Cu") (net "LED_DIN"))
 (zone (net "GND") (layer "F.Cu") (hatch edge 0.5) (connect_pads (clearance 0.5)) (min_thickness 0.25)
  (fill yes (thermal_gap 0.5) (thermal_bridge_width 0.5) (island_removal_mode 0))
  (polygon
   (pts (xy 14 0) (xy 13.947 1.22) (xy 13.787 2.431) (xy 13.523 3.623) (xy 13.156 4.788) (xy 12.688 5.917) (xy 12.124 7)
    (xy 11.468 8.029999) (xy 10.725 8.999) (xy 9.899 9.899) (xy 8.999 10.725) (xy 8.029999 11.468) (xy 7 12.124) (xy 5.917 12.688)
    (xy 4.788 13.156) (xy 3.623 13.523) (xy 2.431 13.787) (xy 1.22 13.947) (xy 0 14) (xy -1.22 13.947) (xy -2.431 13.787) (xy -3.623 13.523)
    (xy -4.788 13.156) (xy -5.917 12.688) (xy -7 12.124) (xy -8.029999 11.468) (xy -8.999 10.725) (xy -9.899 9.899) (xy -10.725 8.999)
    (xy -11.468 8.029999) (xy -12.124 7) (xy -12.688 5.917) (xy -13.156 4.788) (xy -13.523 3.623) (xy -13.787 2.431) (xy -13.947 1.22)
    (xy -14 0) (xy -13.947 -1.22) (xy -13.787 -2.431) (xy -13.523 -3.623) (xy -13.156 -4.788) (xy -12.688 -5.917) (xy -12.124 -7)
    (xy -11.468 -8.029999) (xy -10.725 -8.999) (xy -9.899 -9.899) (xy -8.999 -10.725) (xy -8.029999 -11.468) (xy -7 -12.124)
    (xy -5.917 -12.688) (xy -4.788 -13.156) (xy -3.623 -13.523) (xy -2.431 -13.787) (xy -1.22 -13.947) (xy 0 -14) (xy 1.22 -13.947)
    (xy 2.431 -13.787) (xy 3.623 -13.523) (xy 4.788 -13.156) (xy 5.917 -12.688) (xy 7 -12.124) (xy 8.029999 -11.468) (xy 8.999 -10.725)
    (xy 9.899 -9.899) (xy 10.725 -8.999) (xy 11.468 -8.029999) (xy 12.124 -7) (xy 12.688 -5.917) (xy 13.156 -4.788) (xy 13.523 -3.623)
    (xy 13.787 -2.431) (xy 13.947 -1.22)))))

